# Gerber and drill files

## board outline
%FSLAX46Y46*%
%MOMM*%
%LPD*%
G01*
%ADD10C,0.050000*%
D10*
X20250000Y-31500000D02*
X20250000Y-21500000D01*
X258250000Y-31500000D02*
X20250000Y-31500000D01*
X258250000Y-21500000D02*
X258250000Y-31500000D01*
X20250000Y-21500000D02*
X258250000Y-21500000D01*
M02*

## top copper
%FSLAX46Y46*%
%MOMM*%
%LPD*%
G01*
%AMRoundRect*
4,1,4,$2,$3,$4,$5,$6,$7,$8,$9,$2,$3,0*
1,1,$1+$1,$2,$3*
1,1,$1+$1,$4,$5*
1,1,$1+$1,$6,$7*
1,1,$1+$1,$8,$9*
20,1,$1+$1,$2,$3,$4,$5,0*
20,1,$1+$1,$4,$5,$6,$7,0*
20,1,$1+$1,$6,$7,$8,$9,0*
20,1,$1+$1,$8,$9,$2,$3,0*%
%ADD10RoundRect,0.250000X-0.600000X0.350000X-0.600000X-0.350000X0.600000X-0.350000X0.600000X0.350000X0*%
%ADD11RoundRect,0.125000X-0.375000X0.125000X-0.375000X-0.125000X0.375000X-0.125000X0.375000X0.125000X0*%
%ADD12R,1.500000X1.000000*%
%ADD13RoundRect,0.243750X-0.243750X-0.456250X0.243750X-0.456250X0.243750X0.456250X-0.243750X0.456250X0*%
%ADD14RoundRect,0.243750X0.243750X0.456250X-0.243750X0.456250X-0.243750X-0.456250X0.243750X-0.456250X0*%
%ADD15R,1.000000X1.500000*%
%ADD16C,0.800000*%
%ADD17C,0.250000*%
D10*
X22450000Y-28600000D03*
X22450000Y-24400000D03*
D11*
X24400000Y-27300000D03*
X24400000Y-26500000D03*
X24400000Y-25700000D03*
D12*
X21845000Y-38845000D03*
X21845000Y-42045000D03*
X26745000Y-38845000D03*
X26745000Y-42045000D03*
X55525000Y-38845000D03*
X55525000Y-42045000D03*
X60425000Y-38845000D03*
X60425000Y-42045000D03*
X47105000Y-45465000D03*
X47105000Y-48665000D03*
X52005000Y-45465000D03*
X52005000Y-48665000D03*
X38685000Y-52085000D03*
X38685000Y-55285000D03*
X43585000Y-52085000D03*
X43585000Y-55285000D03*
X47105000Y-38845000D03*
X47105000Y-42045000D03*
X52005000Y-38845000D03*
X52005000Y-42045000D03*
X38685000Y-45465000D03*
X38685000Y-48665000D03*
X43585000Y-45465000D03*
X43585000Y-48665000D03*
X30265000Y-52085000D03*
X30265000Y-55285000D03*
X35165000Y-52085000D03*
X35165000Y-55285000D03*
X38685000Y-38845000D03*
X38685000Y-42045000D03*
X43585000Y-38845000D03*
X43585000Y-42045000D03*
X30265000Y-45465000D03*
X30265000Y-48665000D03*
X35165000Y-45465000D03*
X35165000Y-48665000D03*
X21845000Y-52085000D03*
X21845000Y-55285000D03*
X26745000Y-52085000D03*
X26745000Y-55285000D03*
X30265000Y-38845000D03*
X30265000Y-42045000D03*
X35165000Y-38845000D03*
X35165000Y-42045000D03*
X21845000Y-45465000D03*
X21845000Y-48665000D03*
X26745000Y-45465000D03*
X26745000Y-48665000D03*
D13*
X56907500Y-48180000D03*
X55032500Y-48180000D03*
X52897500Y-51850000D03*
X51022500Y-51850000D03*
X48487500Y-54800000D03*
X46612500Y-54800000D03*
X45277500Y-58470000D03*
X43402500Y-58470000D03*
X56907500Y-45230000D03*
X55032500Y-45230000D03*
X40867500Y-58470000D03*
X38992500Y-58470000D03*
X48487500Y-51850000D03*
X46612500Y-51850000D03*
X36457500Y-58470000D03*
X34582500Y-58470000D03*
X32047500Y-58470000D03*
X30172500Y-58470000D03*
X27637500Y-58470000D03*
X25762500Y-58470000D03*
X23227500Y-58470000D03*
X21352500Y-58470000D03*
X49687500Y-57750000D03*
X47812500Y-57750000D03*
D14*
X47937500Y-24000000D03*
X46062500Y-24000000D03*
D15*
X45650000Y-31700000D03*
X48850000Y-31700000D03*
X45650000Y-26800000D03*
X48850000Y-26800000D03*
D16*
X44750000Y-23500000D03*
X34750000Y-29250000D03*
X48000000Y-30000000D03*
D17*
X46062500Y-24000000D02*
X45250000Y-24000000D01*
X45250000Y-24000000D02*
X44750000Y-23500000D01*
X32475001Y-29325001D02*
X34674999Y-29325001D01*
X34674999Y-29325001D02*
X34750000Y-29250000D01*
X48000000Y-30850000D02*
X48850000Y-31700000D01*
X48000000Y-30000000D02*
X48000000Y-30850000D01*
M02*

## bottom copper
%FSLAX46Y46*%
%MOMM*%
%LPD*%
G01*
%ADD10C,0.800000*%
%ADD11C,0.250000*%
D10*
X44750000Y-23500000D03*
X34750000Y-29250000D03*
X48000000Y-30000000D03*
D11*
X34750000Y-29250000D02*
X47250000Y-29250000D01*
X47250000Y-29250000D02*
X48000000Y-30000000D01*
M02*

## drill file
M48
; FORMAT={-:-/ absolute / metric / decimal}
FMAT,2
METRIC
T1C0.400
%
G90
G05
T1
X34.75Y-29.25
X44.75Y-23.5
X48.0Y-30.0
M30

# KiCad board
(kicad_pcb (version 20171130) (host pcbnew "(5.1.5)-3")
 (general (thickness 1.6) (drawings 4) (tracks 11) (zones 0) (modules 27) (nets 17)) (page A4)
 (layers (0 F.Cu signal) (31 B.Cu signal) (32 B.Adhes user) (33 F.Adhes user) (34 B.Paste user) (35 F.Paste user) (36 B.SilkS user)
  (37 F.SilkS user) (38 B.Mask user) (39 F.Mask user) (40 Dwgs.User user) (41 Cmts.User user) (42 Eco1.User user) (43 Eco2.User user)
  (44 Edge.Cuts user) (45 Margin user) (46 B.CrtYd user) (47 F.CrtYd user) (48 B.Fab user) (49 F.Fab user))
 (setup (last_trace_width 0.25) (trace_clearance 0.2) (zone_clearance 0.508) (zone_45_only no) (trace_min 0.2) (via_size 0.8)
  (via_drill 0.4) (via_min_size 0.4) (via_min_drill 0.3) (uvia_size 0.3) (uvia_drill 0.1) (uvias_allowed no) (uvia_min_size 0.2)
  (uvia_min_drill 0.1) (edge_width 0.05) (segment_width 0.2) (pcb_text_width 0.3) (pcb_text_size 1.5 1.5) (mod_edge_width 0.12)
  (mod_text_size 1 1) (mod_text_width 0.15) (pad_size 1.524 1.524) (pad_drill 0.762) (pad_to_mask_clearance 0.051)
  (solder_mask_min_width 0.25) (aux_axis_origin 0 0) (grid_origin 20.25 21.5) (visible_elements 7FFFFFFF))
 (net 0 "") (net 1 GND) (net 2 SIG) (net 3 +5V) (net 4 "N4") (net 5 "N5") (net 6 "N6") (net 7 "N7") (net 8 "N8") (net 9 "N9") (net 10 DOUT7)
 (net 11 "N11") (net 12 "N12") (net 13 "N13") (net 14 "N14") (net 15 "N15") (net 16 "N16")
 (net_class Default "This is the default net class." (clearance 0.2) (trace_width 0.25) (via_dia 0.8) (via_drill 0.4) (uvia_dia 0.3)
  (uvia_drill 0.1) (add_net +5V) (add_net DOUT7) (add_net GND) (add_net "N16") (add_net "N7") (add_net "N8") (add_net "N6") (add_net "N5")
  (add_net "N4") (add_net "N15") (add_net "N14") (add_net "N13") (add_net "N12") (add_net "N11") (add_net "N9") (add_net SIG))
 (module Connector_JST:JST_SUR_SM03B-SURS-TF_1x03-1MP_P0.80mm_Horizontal (layer F.Cu) (at 23.25 26.5 270)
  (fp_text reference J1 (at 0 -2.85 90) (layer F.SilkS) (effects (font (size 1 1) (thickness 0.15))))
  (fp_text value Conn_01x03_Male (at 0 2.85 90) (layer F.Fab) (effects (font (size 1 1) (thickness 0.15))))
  (pad MP smd roundrect (at 2.1 0.8 270) (size 1.2 1.7) (layers F.Cu F.Paste F.Mask) (roundrect_rratio 0.208333))
  (pad MP smd roundrect (at -2.1 0.8 270) (size 1.2 1.7) (layers F.Cu F.Paste F.Mask) (roundrect_rratio 0.208333))
  (pad 3 smd roundrect (at 0.8 -1.15 270) (size 0.5 1) (layers F.Cu F.Paste F.Mask) (roundrect_rratio 0.25) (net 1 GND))
  (pad 2 smd roundrect (at 0 -1.15 270) (size 0.5 1) (layers F.Cu F.Paste F.Mask) (roundrect_rratio 0.25) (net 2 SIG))
  (pad 1 smd roundrect (at -0.8 -1.15 270) (size 0.5 1) (layers F.Cu F.Paste F.Mask) (roundrect_rratio 0.25) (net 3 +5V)))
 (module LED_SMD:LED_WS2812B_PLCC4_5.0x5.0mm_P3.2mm (layer F.Cu) (at 24.295 40.445)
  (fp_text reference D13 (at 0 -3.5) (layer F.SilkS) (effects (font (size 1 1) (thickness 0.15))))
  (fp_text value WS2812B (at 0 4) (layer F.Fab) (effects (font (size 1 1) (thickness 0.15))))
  (pad 1 smd rect (at -2.45 -1.6) (size 1.5 1) (layers F.Cu F.Paste F.Mask) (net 3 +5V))
  (pad 2 smd rect (at -2.45 1.6) (size 1.5 1) (layers F.Cu F.Paste F.Mask) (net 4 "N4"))
  (pad 4 smd rect (at 2.45 -1.6) (size 1.5 1) (layers F.Cu F.Paste F.Mask) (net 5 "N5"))
  (pad 3 smd rect (at 2.45 1.6) (size 1.5 1) (layers F.Cu F.Paste F.Mask) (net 1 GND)))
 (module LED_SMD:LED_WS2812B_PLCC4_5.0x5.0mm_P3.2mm (layer F.Cu) (at 57.975 40.445)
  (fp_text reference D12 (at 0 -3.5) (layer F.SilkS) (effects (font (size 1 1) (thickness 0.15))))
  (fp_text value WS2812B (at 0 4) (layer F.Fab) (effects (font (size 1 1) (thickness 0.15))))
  (pad 1 smd rect (at -2.45 -1.6) (size 1.5 1) (layers F.Cu F.Paste F.Mask) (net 3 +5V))
  (pad 2 smd rect (at -2.45 1.6) (size 1.5 1) (layers F.Cu F.Paste F.Mask) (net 5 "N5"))
  (pad 4 smd rect (at 2.45 -1.6) (size 1.5 1) (layers F.Cu F.Paste F.Mask) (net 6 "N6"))
  (pad 3 smd rect (at 2.45 1.6) (size 1.5 1) (layers F.Cu F.Paste F.Mask) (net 1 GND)))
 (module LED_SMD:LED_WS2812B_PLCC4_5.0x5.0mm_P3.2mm (layer F.Cu) (at 49.555 47.065)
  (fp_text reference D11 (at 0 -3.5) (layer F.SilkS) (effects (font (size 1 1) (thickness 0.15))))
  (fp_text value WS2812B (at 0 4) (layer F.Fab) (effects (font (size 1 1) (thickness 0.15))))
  (pad 1 smd rect (at -2.45 -1.6) (size 1.5 1) (layers F.Cu F.Paste F.Mask) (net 3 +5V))
  (pad 2 smd rect (at -2.45 1.6) (size 1.5 1) (layers F.Cu F.Paste F.Mask) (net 6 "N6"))
  (pad 4 smd rect (at 2.45 -1.6) (size 1.5 1) (layers F.Cu F.Paste F.Mask) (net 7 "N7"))
  (pad 3 smd rect (at 2.45 1.6) (size 1.5 1) (layers F.Cu F.Paste F.Mask) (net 1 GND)))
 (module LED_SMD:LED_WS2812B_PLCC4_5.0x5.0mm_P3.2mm (layer F.Cu) (at 41.135 53.685)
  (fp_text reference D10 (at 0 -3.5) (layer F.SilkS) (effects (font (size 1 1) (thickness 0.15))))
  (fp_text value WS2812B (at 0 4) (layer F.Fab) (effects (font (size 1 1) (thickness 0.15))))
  (pad 1 smd rect (at -2.45 -1.6) (size 1.5 1) (layers F.Cu F.Paste F.Mask) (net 3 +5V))
  (pad 2 smd rect (at -2.45 1.6) (size 1.5 1) (layers F.Cu F.Paste F.Mask) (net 7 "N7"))
  (pad 4 smd rect (at 2.45 -1.6) (size 1.5 1) (layers F.Cu F.Paste F.Mask) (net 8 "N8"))
  (pad 3 smd rect (at 2.45 1.6) (size 1.5 1) (layers F.Cu F.Paste F.Mask) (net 1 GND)))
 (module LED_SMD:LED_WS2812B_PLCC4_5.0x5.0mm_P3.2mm (layer F.Cu) (at 49.555 40.445)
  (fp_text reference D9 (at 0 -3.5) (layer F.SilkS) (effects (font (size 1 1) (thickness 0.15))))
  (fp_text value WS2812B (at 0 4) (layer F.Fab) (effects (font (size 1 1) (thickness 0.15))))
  (pad 1 smd rect (at -2.45 -1.6) (size 1.5 1) (layers F.Cu F.Paste F.Mask) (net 3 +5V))
  (pad 2 smd rect (at -2.45 1.6) (size 1.5 1) (layers F.Cu F.Paste F.Mask) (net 8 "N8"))
  (pad 4 smd rect (at 2.45 -1.6) (size 1.5 1) (layers F.Cu F.Paste F.Mask) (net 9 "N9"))
  (pad 3 smd rect (at 2.45 1.6) (size 1.5 1) (layers F.Cu F.Paste F.Mask) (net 1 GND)))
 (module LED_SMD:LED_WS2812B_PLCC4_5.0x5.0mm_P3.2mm (layer F.Cu) (at 41.135 47.065)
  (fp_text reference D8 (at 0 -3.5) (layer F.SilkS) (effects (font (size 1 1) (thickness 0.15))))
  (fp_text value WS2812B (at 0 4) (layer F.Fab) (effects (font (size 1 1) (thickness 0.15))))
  (pad 1 smd rect (at -2.45 -1.6) (size 1.5 1) (layers F.Cu F.Paste F.Mask) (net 3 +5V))
  (pad 2 smd rect (at -2.45 1.6) (size 1.5 1) (layers F.Cu F.Paste F.Mask) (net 9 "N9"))
  (pad 4 smd rect (at 2.45 -1.6) (size 1.5 1) (layers F.Cu F.Paste F.Mask) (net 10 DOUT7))
  (pad 3 smd rect (at 2.45 1.6) (size 1.5 1) (layers F.Cu F.Paste F.Mask) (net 1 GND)))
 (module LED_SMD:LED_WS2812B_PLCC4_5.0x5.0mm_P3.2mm (layer F.Cu) (at 32.715 53.685)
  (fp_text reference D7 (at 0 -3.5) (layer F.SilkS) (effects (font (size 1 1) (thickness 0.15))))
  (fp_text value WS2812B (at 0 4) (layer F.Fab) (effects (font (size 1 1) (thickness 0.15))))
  (pad 1 smd rect (at -2.45 -1.6) (size 1.5 1) (layers F.Cu F.Paste F.Mask) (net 3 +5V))
  (pad 2 smd rect (at -2.45 1.6) (size 1.5 1) (layers F.Cu F.Paste F.Mask) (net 10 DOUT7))
  (pad 4 smd rect (at 2.45 -1.6) (size 1.5 1) (layers F.Cu F.Paste F.Mask) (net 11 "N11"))
  (pad 3 smd rect (at 2.45 1.6) (size 1.5 1) (layers F.Cu F.Paste F.Mask) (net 1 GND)))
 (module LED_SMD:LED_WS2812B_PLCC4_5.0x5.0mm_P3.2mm (layer F.Cu) (at 41.135 40.445)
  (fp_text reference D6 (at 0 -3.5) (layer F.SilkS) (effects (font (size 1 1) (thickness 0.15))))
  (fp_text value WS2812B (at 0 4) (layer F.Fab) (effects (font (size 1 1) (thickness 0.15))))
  (pad 1 smd rect (at -2.45 -1.6) (size 1.5 1) (layers F.Cu F.Paste F.Mask) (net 3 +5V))
  (pad 2 smd rect (at -2.45 1.6) (size 1.5 1) (layers F.Cu F.Paste F.Mask) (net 11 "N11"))
  (pad 4 smd rect (at 2.45 -1.6) (size 1.5 1) (layers F.Cu F.Paste F.Mask) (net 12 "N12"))
  (pad 3 smd rect (at 2.45 1.6) (size 1.5 1) (layers F.Cu F.Paste F.Mask) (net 1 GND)))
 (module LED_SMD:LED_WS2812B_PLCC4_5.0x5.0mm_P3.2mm (layer F.Cu) (at 32.715 47.065)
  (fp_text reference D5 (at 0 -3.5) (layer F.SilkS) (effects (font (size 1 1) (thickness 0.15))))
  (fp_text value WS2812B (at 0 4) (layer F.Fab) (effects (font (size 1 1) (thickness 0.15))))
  (pad 1 smd rect (at -2.45 -1.6) (size 1.5 1) (layers F.Cu F.Paste F.Mask) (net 3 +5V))
  (pad 2 smd rect (at -2.45 1.6) (size 1.5 1) (layers F.Cu F.Paste F.Mask) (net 12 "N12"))
  (pad 4 smd rect (at 2.45 -1.6) (size 1.5 1) (layers F.Cu F.Paste F.Mask) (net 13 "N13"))
  (pad 3 smd rect (at 2.45 1.6) (size 1.5 1) (layers F.Cu F.Paste F.Mask) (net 1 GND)))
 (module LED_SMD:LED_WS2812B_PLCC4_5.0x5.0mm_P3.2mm (layer F.Cu) (at 24.295 53.685)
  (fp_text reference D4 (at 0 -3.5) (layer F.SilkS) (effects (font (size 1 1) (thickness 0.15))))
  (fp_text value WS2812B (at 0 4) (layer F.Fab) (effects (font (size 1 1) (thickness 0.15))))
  (pad 1 smd rect (at -2.45 -1.6) (size 1.5 1) (layers F.Cu F.Paste F.Mask) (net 3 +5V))
  (pad 2 smd rect (at -2.45 1.6) (size 1.5 1) (layers F.Cu F.Paste F.Mask) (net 13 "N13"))
  (pad 4 smd rect (at 2.45 -1.6) (size 1.5 1) (layers F.Cu F.Paste F.Mask) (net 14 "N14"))
  (pad 3 smd rect (at 2.45 1.6) (size 1.5 1) (layers F.Cu F.Paste F.Mask) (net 1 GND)))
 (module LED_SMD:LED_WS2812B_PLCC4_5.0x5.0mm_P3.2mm (layer F.Cu) (at 32.715 40.445)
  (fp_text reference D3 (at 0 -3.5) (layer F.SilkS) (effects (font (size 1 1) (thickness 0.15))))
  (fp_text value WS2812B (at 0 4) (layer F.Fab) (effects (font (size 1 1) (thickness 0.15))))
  (pad 1 smd rect (at -2.45 -1.6) (size 1.5 1) (layers F.Cu F.Paste F.Mask) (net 3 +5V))
  (pad 2 smd rect (at -2.45 1.6) (size 1.5 1) (layers F.Cu F.Paste F.Mask) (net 14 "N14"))
  (pad 4 smd rect (at 2.45 -1.6) (size 1.5 1) (layers F.Cu F.Paste F.Mask) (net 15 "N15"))
  (pad 3 smd rect (at 2.45 1.6) (size 1.5 1) (layers F.Cu F.Paste F.Mask) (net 1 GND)))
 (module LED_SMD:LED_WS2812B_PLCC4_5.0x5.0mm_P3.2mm (layer F.Cu) (at 24.295 47.065)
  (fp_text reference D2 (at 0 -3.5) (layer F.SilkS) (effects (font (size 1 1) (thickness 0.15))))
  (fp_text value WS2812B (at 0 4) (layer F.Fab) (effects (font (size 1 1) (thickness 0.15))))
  (pad 1 smd rect (at -2.45 -1.6) (size 1.5 1) (layers F.Cu F.Paste F.Mask) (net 3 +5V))
  (pad 2 smd rect (at -2.45 1.6) (size 1.5 1) (layers F.Cu F.Paste F.Mask) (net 15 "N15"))
  (pad 4 smd rect (at 2.45 -1.6) (size 1.5 1) (layers F.Cu F.Paste F.Mask) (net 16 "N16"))
  (pad 3 smd rect (at 2.45 1.6) (size 1.5 1) (layers F.Cu F.Paste F.Mask) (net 1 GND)))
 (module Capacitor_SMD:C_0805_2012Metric (layer F.Cu) (at 55.97 48.18)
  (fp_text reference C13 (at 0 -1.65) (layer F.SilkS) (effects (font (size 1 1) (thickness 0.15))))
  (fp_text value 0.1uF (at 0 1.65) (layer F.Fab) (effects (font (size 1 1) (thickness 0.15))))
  (pad 2 smd roundrect (at 0.9375 0) (size 0.975 1.4) (layers F.Cu F.Paste F.Mask) (roundrect_rratio 0.25) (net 1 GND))
  (pad 1 smd roundrect (at -0.9375 0) (size 0.975 1.4) (layers F.Cu F.Paste F.Mask) (roundrect_rratio 0.25) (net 3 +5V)))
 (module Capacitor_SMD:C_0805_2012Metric (layer F.Cu) (at 51.96 51.85)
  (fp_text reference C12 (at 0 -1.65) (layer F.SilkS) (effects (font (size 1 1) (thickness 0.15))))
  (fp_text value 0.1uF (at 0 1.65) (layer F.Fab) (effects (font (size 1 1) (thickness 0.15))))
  (pad 2 smd roundrect (at 0.9375 0) (size 0.975 1.4) (layers F.Cu F.Paste F.Mask) (roundrect_rratio 0.25) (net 1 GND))
  (pad 1 smd roundrect (at -0.9375 0) (size 0.975 1.4) (layers F.Cu F.Paste F.Mask) (roundrect_rratio 0.25) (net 3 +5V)))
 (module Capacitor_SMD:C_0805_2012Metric (layer F.Cu) (at 47.55 54.8)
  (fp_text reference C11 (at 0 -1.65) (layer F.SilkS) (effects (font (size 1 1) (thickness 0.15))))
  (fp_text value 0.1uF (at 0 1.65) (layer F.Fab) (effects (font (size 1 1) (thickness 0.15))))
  (pad 2 smd roundrect (at 0.9375 0) (size 0.975 1.4) (layers F.Cu F.Paste F.Mask) (roundrect_rratio 0.25) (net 1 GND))
  (pad 1 smd roundrect (at -0.9375 0) (size 0.975 1.4) (layers F.Cu F.Paste F.Mask) (roundrect_rratio 0.25) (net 3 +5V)))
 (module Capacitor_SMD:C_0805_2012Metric (layer F.Cu) (at 44.34 58.47)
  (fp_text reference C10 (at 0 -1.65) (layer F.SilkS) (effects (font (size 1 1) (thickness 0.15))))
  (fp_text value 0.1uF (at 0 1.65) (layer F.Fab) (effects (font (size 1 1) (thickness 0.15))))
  (pad 2 smd roundrect (at 0.9375 0) (size 0.975 1.4) (layers F.Cu F.Paste F.Mask) (roundrect_rratio 0.25) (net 1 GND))
  (pad 1 smd roundrect (at -0.9375 0) (size 0.975 1.4) (layers F.Cu F.Paste F.Mask) (roundrect_rratio 0.25) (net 3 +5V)))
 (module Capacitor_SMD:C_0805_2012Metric (layer F.Cu) (at 55.97 45.23)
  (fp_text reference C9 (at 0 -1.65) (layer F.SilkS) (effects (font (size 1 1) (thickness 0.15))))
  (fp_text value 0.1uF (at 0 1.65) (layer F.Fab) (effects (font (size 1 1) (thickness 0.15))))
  (pad 2 smd roundrect (at 0.9375 0) (size 0.975 1.4) (layers F.Cu F.Paste F.Mask) (roundrect_rratio 0.25) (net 1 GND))
  (pad 1 smd roundrect (at -0.9375 0) (size 0.975 1.4) (layers F.Cu F.Paste F.Mask) (roundrect_rratio 0.25) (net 3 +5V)))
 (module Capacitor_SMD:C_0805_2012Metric (layer F.Cu) (at 39.93 58.47)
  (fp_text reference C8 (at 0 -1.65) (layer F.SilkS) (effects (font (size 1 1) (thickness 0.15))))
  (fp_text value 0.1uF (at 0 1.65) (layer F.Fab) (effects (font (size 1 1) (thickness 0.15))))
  (pad 2 smd roundrect (at 0.9375 0) (size 0.975 1.4) (layers F.Cu F.Paste F.Mask) (roundrect_rratio 0.25) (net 1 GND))
  (pad 1 smd roundrect (at -0.9375 0) (size 0.975 1.4) (layers F.Cu F.Paste F.Mask) (roundrect_rratio 0.25) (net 3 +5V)))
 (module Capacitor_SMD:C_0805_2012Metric (layer F.Cu) (at 47.55 51.85)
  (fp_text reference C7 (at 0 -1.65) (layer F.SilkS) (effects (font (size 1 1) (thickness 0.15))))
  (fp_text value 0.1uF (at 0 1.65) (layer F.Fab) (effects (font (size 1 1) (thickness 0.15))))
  (pad 2 smd roundrect (at 0.9375 0) (size 0.975 1.4) (layers F.Cu F.Paste F.Mask) (roundrect_rratio 0.25) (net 1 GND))
  (pad 1 smd roundrect (at -0.9375 0) (size 0.975 1.4) (layers F.Cu F.Paste F.Mask) (roundrect_rratio 0.25) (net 3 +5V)))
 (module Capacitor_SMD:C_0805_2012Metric (layer F.Cu) (at 35.52 58.47)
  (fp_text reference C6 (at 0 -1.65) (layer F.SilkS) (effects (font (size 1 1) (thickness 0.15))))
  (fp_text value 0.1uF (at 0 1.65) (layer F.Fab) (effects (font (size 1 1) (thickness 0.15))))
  (pad 2 smd roundrect (at 0.9375 0) (size 0.975 1.4) (layers F.Cu F.Paste F.Mask) (roundrect_rratio 0.25) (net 1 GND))
  (pad 1 smd roundrect (at -0.9375 0) (size 0.975 1.4) (layers F.Cu F.Paste F.Mask) (roundrect_rratio 0.25) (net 3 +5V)))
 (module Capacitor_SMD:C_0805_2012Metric (layer F.Cu) (at 31.11 58.47)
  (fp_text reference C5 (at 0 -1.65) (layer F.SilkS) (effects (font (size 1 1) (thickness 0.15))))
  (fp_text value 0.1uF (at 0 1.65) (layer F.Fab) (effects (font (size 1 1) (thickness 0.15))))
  (pad 2 smd roundrect (at 0.9375 0) (size 0.975 1.4) (layers F.Cu F.Paste F.Mask) (roundrect_rratio 0.25) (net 1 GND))
  (pad 1 smd roundrect (at -0.9375 0) (size 0.975 1.4) (layers F.Cu F.Paste F.Mask) (roundrect_rratio 0.25) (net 3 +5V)))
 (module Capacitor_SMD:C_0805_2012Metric (layer F.Cu) (at 26.7 58.47)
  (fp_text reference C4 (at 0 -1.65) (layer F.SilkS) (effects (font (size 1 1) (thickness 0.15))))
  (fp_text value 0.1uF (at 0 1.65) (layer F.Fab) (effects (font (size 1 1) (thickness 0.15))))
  (pad 2 smd roundrect (at 0.9375 0) (size 0.975 1.4) (layers F.Cu F.Paste F.Mask) (roundrect_rratio 0.25) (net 1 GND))
  (pad 1 smd roundrect (at -0.9375 0) (size 0.975 1.4) (layers F.Cu F.Paste F.Mask) (roundrect_rratio 0.25) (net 3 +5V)))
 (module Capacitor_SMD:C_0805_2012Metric (layer F.Cu) (at 22.29 58.47)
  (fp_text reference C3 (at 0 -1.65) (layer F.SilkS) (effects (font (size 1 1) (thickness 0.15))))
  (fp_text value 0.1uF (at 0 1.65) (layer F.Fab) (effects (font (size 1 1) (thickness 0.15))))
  (pad 2 smd roundrect (at 0.9375 0) (size 0.975 1.4) (layers F.Cu F.Paste F.Mask) (roundrect_rratio 0.25) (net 1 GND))
  (pad 1 smd roundrect (at -0.9375 0) (size 0.975 1.4) (layers F.Cu F.Paste F.Mask) (roundrect_rratio 0.25) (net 3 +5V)))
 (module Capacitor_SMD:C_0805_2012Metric (layer F.Cu) (at 48.75 57.75)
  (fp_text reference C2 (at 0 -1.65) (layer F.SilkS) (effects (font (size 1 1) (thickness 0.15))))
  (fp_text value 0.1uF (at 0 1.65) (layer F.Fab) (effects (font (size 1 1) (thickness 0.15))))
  (pad 2 smd roundrect (at 0.9375 0) (size 0.975 1.4) (layers F.Cu F.Paste F.Mask) (roundrect_rratio 0.25) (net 1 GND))
  (pad 1 smd roundrect (at -0.9375 0) (size 0.975 1.4) (layers F.Cu F.Paste F.Mask) (roundrect_rratio 0.25) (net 3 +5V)))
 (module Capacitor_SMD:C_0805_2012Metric (layer F.Cu) (at 47 24 180)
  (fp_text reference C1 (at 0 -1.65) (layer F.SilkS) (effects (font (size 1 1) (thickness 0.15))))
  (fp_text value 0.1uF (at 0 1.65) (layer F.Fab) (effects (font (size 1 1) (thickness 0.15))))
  (pad 1 smd roundrect (at -0.9375 0 180) (size 0.975 1.4) (layers F.Cu F.Paste F.Mask) (roundrect_rratio 0.25) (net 3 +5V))
  (pad 2 smd roundrect (at 0.9375 0 180) (size 0.975 1.4) (layers F.Cu F.Paste F.Mask) (roundrect_rratio 0.25) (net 1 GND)))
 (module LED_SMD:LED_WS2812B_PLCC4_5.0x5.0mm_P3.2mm (layer F.Cu) (at 47.25 29.25 270)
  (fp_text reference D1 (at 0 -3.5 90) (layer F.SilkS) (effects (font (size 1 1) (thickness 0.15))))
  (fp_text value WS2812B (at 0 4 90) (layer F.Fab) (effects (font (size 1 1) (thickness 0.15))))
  (pad 3 smd rect (at 2.45 1.6 270) (size 1.5 1) (layers F.Cu F.Paste F.Mask) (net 1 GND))
  (pad 4 smd rect (at 2.45 -1.6 270) (size 1.5 1) (layers F.Cu F.Paste F.Mask) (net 2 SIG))
  (pad 2 smd rect (at -2.45 1.6 270) (size 1.5 1) (layers F.Cu F.Paste F.Mask) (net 16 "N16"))
  (pad 1 smd rect (at -2.45 -1.6 270) (size 1.5 1) (layers F.Cu F.Paste F.Mask) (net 3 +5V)))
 (gr_line (start 20.25 31.5) (end 20.25 21.5) (layer Edge.Cuts) (width 0.05))
 (gr_line (start 258.25 31.5) (end 20.25 31.5) (layer Edge.Cuts) (width 0.05))
 (gr_line (start 258.25 21.5) (end 258.25 31.5) (layer Edge.Cuts) (width 0.05))
 (gr_line (start 20.25 21.5) (end 258.25 21.5) (layer Edge.Cuts) (width 0.05))
 (via (at 44.75 23.5) (size 0.8) (drill 0.4) (layers F.Cu B.Cu) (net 1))
 (segment (start 46.0625 24) (end 45.25 24) (width 0.25) (layer F.Cu) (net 1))
 (segment (start 45.25 24) (end 44.75 23.5) (width 0.25) (layer F.Cu) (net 1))
 (via (at 34.75 29.25) (size 0.8) (drill 0.4) (layers F.Cu B.Cu) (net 2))
 (segment (start 32.475001 29.325001) (end 34.674999 29.325001) (width 0.25) (layer F.Cu) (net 2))
 (segment (start 34.674999 29.325001) (end 34.75 29.25) (width 0.25) (layer F.Cu) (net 2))
 (segment (start 34.75 29.25) (end 47.25 29.25) (width 0.25) (layer B.Cu) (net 2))
 (via (at 48 30) (size 0.8) (drill 0.4) (layers F.Cu B.Cu) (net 2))
 (segment (start 47.25 29.25) (end 48 30) (width 0.25) (layer B.Cu) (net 2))
 (segment (start 48 30.85) (end 48.85 31.7) (width 0.25) (layer F.Cu) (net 2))
 (segment (start 48 30) (end 48 30.85) (width 0.25) (layer F.Cu) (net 2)))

